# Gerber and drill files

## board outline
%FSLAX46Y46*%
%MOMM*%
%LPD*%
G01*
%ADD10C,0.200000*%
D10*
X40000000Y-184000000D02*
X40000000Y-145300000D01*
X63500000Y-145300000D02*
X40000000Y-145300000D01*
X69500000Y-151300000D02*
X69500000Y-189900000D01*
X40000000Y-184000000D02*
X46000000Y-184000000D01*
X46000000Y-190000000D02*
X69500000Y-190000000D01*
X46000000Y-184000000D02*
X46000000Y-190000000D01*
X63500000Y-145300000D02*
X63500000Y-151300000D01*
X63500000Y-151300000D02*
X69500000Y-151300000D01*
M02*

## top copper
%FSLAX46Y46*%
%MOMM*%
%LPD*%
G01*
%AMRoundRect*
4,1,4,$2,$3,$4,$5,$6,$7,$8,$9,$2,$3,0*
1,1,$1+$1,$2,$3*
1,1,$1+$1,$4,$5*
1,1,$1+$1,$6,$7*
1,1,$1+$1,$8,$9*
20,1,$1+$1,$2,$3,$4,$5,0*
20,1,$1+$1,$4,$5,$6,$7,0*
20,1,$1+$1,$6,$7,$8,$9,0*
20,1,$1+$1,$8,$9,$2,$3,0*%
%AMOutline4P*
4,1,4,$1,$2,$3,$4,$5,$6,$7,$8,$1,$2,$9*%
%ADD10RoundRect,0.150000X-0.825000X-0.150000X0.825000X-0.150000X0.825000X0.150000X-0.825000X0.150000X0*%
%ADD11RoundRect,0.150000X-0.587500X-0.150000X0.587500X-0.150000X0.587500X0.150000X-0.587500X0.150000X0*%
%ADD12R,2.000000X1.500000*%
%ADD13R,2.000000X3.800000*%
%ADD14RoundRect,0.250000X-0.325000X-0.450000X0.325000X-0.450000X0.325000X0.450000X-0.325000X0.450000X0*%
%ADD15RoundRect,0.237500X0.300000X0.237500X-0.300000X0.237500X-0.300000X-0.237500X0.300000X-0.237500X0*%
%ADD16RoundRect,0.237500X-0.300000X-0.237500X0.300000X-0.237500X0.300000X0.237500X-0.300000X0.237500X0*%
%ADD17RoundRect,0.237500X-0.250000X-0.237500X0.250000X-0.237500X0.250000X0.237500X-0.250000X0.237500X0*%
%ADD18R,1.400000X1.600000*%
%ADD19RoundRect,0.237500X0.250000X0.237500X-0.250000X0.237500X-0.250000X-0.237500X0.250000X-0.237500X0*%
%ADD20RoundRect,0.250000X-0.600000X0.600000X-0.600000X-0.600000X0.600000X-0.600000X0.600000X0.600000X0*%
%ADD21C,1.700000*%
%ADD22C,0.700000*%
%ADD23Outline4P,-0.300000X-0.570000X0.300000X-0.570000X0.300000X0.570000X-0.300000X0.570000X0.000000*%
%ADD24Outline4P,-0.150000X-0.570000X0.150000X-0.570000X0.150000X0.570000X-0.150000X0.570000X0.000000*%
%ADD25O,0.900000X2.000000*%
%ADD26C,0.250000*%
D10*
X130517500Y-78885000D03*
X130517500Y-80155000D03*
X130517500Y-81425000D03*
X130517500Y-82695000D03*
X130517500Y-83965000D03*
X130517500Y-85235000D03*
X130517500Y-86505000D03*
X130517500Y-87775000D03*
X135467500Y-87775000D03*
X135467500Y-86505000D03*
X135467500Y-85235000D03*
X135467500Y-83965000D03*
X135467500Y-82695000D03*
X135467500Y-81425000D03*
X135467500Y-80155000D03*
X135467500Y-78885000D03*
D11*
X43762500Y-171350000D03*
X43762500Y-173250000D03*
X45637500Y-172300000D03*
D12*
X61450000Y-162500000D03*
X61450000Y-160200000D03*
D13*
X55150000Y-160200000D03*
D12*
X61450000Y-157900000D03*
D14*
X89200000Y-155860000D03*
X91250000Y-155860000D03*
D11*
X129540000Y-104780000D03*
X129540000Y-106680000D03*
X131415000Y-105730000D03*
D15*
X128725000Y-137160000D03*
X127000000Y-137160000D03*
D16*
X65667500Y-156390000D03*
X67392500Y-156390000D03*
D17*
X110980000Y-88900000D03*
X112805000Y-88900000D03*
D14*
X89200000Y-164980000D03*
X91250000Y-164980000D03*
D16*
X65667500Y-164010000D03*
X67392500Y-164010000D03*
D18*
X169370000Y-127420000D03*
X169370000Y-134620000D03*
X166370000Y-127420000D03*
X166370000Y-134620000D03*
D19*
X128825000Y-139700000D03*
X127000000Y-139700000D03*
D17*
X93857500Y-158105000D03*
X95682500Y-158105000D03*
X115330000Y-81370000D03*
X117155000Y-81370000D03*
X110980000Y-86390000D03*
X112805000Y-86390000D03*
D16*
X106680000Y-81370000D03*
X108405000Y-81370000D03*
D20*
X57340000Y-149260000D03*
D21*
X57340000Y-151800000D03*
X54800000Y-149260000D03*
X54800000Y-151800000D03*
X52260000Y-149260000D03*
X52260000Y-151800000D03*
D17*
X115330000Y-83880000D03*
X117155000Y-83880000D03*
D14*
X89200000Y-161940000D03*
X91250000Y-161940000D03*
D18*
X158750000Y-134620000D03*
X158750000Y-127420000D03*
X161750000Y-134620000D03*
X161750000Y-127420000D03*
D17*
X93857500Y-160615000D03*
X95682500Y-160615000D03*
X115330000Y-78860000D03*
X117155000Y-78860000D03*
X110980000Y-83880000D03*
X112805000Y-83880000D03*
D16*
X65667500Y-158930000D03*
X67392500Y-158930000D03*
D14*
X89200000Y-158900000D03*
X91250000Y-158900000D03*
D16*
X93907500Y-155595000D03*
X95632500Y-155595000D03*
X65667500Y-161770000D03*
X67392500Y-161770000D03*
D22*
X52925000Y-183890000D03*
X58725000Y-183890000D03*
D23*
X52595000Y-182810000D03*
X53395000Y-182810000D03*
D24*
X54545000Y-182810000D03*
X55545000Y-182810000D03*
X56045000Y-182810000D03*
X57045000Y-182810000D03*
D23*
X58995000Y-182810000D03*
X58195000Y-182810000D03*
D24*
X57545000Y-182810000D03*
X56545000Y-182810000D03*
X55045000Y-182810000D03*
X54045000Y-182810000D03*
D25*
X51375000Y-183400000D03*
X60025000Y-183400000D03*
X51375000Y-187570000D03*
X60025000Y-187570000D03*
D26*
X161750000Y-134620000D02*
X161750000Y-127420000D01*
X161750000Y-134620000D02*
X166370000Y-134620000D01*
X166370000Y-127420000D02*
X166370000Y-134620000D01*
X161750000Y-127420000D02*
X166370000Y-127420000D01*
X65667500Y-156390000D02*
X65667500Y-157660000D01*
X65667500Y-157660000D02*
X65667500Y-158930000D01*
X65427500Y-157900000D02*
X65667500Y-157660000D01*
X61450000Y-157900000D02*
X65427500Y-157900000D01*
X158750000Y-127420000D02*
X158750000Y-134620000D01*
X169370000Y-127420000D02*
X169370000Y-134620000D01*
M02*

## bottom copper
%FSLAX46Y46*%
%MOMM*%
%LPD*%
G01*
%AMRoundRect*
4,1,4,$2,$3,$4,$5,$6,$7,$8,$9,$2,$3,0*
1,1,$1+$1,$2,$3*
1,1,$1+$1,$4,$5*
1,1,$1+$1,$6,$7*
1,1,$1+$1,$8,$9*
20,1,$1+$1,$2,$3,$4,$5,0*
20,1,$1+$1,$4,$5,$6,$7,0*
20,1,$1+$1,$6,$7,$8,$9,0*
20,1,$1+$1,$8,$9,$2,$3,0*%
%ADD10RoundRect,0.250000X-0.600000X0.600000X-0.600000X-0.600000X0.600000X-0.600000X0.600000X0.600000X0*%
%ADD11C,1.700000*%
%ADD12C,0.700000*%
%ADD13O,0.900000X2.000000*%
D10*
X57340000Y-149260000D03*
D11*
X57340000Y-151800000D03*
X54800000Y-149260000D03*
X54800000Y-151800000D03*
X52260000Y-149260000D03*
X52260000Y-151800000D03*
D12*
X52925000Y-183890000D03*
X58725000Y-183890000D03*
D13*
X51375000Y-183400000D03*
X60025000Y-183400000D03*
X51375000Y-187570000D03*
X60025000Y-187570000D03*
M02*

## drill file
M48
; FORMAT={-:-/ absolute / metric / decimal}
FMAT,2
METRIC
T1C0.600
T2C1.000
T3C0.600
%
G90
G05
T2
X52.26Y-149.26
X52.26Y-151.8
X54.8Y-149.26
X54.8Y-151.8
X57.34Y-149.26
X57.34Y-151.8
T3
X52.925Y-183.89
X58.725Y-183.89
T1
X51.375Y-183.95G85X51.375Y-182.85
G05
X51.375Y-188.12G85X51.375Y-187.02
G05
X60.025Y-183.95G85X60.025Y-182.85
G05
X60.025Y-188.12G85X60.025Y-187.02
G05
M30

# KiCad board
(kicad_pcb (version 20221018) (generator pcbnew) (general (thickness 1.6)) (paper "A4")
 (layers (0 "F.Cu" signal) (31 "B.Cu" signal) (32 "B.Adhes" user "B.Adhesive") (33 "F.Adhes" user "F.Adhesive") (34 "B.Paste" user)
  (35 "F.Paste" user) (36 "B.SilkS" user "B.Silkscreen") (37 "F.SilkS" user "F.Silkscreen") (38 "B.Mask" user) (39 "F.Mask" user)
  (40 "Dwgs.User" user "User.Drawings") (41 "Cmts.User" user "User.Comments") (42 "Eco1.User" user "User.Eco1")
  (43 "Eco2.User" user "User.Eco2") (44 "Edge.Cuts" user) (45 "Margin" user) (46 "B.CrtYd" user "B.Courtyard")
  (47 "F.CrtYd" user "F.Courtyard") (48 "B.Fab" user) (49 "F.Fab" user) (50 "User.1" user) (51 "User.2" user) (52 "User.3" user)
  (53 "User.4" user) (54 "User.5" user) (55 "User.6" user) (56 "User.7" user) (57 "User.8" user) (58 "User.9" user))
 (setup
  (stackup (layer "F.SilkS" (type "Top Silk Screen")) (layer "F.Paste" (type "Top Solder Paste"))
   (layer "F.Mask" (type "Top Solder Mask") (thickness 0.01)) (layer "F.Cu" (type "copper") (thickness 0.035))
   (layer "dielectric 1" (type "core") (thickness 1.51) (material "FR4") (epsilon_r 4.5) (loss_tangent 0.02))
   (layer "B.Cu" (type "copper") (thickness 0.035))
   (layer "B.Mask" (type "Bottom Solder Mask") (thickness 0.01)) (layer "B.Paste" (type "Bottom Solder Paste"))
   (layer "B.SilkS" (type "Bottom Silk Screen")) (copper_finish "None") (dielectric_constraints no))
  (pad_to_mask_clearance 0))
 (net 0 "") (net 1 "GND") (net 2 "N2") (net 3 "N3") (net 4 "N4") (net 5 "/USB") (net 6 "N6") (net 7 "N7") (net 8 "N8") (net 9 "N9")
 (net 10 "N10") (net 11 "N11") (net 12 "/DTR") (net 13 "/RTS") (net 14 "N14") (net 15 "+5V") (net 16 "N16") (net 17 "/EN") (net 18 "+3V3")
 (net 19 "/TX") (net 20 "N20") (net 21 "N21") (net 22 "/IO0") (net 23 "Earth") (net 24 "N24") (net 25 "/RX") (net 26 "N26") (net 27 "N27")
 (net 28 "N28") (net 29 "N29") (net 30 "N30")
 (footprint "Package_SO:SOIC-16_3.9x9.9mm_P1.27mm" (layer "F.Cu") (at 132.9925 83.33)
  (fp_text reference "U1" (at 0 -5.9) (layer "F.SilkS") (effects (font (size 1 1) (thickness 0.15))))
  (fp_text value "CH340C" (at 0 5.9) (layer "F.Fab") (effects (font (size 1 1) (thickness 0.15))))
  (pad "1" smd roundrect (at -2.475 -4.445) (size 1.95 0.6) (layers "F.Cu" "F.Paste" "F.Mask") (roundrect_rratio 0.25) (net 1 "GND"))
  (pad "2" smd roundrect (at -2.475 -3.175) (size 1.95 0.6) (layers "F.Cu" "F.Paste" "F.Mask") (roundrect_rratio 0.25) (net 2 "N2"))
  (pad "3" smd roundrect (at -2.475 -1.905) (size 1.95 0.6) (layers "F.Cu" "F.Paste" "F.Mask") (roundrect_rratio 0.25) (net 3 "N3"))
  (pad "4" smd roundrect (at -2.475 -0.635) (size 1.95 0.6) (layers "F.Cu" "F.Paste" "F.Mask") (roundrect_rratio 0.25) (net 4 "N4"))
  (pad "5" smd roundrect (at -2.475 0.635) (size 1.95 0.6) (layers "F.Cu" "F.Paste" "F.Mask") (roundrect_rratio 0.25) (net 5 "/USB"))
  (pad "6" smd roundrect (at -2.475 1.905) (size 1.95 0.6) (layers "F.Cu" "F.Paste" "F.Mask") (roundrect_rratio 0.25) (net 5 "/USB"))
  (pad "7" smd roundrect (at -2.475 3.175) (size 1.95 0.6) (layers "F.Cu" "F.Paste" "F.Mask") (roundrect_rratio 0.25) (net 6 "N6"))
  (pad "8" smd roundrect (at -2.475 4.445) (size 1.95 0.6) (layers "F.Cu" "F.Paste" "F.Mask") (roundrect_rratio 0.25) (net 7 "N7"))
  (pad "9" smd roundrect (at 2.475 4.445) (size 1.95 0.6) (layers "F.Cu" "F.Paste" "F.Mask") (roundrect_rratio 0.25) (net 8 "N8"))
  (pad "10" smd roundrect (at 2.475 3.175) (size 1.95 0.6) (layers "F.Cu" "F.Paste" "F.Mask") (roundrect_rratio 0.25) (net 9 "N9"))
  (pad "11" smd roundrect (at 2.475 1.905) (size 1.95 0.6) (layers "F.Cu" "F.Paste" "F.Mask") (roundrect_rratio 0.25) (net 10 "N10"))
  (pad "12" smd roundrect (at 2.475 0.635) (size 1.95 0.6) (layers "F.Cu" "F.Paste" "F.Mask") (roundrect_rratio 0.25) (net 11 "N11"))
  (pad "13" smd roundrect (at 2.475 -0.635) (size 1.95 0.6) (layers "F.Cu" "F.Paste" "F.Mask") (roundrect_rratio 0.25) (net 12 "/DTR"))
  (pad "14" smd roundrect (at 2.475 -1.905) (size 1.95 0.6) (layers "F.Cu" "F.Paste" "F.Mask") (roundrect_rratio 0.25) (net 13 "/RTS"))
  (pad "15" smd roundrect (at 2.475 -3.175) (size 1.95 0.6) (layers "F.Cu" "F.Paste" "F.Mask") (roundrect_rratio 0.25) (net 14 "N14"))
  (pad "16" smd roundrect (at 2.475 -4.445) (size 1.95 0.6) (layers "F.Cu" "F.Paste" "F.Mask") (roundrect_rratio 0.25) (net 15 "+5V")))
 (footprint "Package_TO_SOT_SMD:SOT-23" (layer "F.Cu") (at 44.7 172.3)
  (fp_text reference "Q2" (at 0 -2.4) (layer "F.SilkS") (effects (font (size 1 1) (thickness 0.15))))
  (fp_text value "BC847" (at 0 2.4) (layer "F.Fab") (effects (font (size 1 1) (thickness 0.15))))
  (pad "1" smd roundrect (at -0.9375 -0.95) (size 1.475 0.6) (layers "F.Cu" "F.Paste" "F.Mask") (roundrect_rratio 0.25) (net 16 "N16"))
  (pad "2" smd roundrect (at -0.9375 0.95) (size 1.475 0.6) (layers "F.Cu" "F.Paste" "F.Mask") (roundrect_rratio 0.25) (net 13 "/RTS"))
  (pad "3" smd roundrect (at 0.9375 0) (size 1.475 0.6) (layers "F.Cu" "F.Paste" "F.Mask") (roundrect_rratio 0.25) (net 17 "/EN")))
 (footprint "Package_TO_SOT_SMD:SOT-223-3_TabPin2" (layer "F.Cu") (at 58.3 160.2 180)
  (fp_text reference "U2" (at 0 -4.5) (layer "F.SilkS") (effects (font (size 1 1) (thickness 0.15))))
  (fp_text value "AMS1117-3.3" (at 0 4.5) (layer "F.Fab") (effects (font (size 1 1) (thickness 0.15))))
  (pad "1" smd rect (at -3.15 -2.3 180) (size 2 1.5) (layers "F.Cu" "F.Paste" "F.Mask") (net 1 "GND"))
  (pad "2" smd rect (at -3.15 0 180) (size 2 1.5) (layers "F.Cu" "F.Paste" "F.Mask") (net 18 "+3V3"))
  (pad "2" smd rect (at 3.15 0 180) (size 2 3.8) (layers "F.Cu" "F.Paste" "F.Mask") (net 18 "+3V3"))
  (pad "3" smd rect (at -3.15 2.3 180) (size 2 1.5) (layers "F.Cu" "F.Paste" "F.Mask") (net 15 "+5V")))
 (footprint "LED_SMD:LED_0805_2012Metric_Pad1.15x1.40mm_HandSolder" (layer "F.Cu") (at 90.225 155.86)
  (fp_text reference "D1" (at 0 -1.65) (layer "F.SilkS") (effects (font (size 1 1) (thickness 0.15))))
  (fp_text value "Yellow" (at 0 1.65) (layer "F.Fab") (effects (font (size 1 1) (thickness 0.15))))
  (pad "1" smd roundrect (at -1.025 0) (size 1.15 1.4) (layers "F.Cu" "F.Paste" "F.Mask") (roundrect_rratio 0.217391) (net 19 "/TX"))
  (pad "2" smd roundrect (at 1.025 0) (size 1.15 1.4) (layers "F.Cu" "F.Paste" "F.Mask") (roundrect_rratio 0.217391) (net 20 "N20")))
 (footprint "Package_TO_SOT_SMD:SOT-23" (layer "F.Cu") (at 130.4775 105.73)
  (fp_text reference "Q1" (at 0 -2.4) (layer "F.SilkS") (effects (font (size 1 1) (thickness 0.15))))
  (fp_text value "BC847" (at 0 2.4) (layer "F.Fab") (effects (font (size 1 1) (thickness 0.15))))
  (pad "1" smd roundrect (at -0.9375 -0.95) (size 1.475 0.6) (layers "F.Cu" "F.Paste" "F.Mask") (roundrect_rratio 0.25) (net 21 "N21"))
  (pad "2" smd roundrect (at -0.9375 0.95) (size 1.475 0.6) (layers "F.Cu" "F.Paste" "F.Mask") (roundrect_rratio 0.25) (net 12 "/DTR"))
  (pad "3" smd roundrect (at 0.9375 0) (size 1.475 0.6) (layers "F.Cu" "F.Paste" "F.Mask") (roundrect_rratio 0.25) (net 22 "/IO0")))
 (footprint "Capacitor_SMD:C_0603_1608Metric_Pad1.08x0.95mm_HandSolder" (layer "F.Cu") (at 127.8625 137.16 180)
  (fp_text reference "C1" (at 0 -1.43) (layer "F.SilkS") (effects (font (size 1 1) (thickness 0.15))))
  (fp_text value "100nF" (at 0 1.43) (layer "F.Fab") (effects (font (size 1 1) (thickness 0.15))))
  (pad "1" smd roundrect (at -0.8625 0 180) (size 1.075 0.95) (layers "F.Cu" "F.Paste" "F.Mask") (roundrect_rratio 0.25) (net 1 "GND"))
  (pad "2" smd roundrect (at 0.8625 0 180) (size 1.075 0.95) (layers "F.Cu" "F.Paste" "F.Mask") (roundrect_rratio 0.25) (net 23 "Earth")))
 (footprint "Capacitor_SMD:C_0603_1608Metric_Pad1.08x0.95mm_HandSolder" (layer "F.Cu") (at 66.53 156.39)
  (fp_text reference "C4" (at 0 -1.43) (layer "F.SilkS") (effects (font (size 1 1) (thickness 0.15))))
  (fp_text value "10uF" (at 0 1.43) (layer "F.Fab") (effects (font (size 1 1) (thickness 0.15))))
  (pad "1" smd roundrect (at -0.8625 0) (size 1.075 0.95) (layers "F.Cu" "F.Paste" "F.Mask") (roundrect_rratio 0.25) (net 15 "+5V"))
  (pad "2" smd roundrect (at 0.8625 0) (size 1.075 0.95) (layers "F.Cu" "F.Paste" "F.Mask") (roundrect_rratio 0.25) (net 1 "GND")))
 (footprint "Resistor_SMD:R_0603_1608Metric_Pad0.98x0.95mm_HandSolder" (layer "F.Cu") (at 111.8925 88.9)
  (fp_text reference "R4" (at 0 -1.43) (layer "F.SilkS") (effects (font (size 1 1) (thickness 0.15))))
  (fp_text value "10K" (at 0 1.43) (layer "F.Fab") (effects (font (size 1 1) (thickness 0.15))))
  (pad "1" smd roundrect (at -0.9125 0) (size 0.975 0.95) (layers "F.Cu" "F.Paste" "F.Mask") (roundrect_rratio 0.25) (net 22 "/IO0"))
  (pad "2" smd roundrect (at 0.9125 0) (size 0.975 0.95) (layers "F.Cu" "F.Paste" "F.Mask") (roundrect_rratio 0.25) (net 18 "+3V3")))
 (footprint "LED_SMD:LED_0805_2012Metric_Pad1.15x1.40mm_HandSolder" (layer "F.Cu") (at 90.225 164.98)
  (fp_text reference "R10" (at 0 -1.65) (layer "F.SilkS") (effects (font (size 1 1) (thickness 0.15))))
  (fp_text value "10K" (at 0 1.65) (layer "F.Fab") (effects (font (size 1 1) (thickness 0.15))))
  (pad "1" smd roundrect (at -1.025 0) (size 1.15 1.4) (layers "F.Cu" "F.Paste" "F.Mask") (roundrect_rratio 0.217391) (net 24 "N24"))
  (pad "2" smd roundrect (at 1.025 0) (size 1.15 1.4) (layers "F.Cu" "F.Paste" "F.Mask") (roundrect_rratio 0.217391) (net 18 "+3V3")))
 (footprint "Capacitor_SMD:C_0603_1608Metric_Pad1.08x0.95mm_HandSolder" (layer "F.Cu") (at 66.53 164.01)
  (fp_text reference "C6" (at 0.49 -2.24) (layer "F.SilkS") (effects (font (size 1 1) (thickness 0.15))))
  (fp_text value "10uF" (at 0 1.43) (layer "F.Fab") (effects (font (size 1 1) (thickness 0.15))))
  (pad "1" smd roundrect (at -0.8625 0) (size 1.075 0.95) (layers "F.Cu" "F.Paste" "F.Mask") (roundrect_rratio 0.25) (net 18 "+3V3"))
  (pad "2" smd roundrect (at 0.8625 0) (size 1.075 0.95) (layers "F.Cu" "F.Paste" "F.Mask") (roundrect_rratio 0.25) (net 1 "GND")))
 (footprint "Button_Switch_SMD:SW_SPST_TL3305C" (layer "F.Cu") (at 167.87 131.02 -90)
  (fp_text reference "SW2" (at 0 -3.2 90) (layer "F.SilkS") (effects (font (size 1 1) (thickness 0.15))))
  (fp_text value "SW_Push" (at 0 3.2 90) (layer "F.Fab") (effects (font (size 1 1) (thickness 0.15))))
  (pad "1" smd rect (at -3.6 -1.5 270) (size 1.6 1.4) (layers "F.Cu" "F.Paste" "F.Mask") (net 17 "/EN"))
  (pad "1" smd rect (at 3.6 -1.5 270) (size 1.6 1.4) (layers "F.Cu" "F.Paste" "F.Mask") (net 17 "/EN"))
  (pad "2" smd rect (at -3.6 1.5 270) (size 1.6 1.4) (layers "F.Cu" "F.Paste" "F.Mask") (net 1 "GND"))
  (pad "2" smd rect (at 3.6 1.5 270) (size 1.6 1.4) (layers "F.Cu" "F.Paste" "F.Mask") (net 1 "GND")))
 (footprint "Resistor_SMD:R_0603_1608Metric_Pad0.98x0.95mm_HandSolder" (layer "F.Cu") (at 127.9125 139.7 180)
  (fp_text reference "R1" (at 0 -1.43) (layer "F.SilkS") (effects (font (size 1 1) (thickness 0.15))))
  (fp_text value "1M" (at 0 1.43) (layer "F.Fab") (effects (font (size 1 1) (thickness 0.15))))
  (pad "1" smd roundrect (at -0.9125 0 180) (size 0.975 0.95) (layers "F.Cu" "F.Paste" "F.Mask") (roundrect_rratio 0.25) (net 1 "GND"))
  (pad "2" smd roundrect (at 0.9125 0 180) (size 0.975 0.95) (layers "F.Cu" "F.Paste" "F.Mask") (roundrect_rratio 0.25) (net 23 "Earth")))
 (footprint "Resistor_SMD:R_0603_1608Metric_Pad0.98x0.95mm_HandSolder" (layer "F.Cu") (at 94.77 158.105)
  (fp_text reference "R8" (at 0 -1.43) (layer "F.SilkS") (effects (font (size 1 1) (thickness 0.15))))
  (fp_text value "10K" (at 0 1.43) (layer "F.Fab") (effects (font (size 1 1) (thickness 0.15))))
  (pad "1" smd roundrect (at -0.9125 0) (size 0.975 0.95) (layers "F.Cu" "F.Paste" "F.Mask") (roundrect_rratio 0.25) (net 20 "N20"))
  (pad "2" smd roundrect (at 0.9125 0) (size 0.975 0.95) (layers "F.Cu" "F.Paste" "F.Mask") (roundrect_rratio 0.25) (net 18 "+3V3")))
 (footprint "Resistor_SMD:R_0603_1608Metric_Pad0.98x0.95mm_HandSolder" (layer "F.Cu") (at 116.2425 81.37)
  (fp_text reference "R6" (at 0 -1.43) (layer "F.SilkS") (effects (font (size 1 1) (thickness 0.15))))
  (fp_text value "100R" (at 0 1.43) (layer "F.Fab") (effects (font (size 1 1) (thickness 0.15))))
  (pad "1" smd roundrect (at -0.9125 0) (size 0.975 0.95) (layers "F.Cu" "F.Paste" "F.Mask") (roundrect_rratio 0.25) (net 2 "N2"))
  (pad "2" smd roundrect (at 0.9125 0) (size 0.975 0.95) (layers "F.Cu" "F.Paste" "F.Mask") (roundrect_rratio 0.25) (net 19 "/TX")))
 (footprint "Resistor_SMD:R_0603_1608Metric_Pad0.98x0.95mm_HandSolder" (layer "F.Cu") (at 111.8925 86.39)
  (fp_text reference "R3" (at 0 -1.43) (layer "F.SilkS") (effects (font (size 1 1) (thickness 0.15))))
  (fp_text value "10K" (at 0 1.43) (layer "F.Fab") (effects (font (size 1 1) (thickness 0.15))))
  (pad "1" smd roundrect (at -0.9125 0) (size 0.975 0.95) (layers "F.Cu" "F.Paste" "F.Mask") (roundrect_rratio 0.25) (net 12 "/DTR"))
  (pad "2" smd roundrect (at 0.9125 0) (size 0.975 0.95) (layers "F.Cu" "F.Paste" "F.Mask") (roundrect_rratio 0.25) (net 16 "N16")))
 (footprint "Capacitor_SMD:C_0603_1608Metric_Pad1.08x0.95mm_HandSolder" (layer "F.Cu") (at 107.5425 81.37)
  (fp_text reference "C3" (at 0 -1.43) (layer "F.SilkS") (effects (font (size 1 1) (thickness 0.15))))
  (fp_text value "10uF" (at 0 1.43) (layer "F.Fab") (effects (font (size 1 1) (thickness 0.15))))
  (pad "1" smd roundrect (at -0.8625 0) (size 1.075 0.95) (layers "F.Cu" "F.Paste" "F.Mask") (roundrect_rratio 0.25) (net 15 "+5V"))
  (pad "2" smd roundrect (at 0.8625 0) (size 1.075 0.95) (layers "F.Cu" "F.Paste" "F.Mask") (roundrect_rratio 0.25) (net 1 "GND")))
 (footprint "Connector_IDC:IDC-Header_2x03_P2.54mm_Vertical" (layer "F.Cu") (at 57.34 149.26 -90)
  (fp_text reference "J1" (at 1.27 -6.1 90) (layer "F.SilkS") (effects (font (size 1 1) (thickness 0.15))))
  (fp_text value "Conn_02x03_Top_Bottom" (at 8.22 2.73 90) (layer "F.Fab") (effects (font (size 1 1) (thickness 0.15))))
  (pad "1" thru_hole roundrect (at 0 0 270) (size 1.7 1.7) (drill 1) (layers "*.Cu" "*.Mask") (roundrect_rratio 0.147059) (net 18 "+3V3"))
  (pad "2" thru_hole circle (at 2.54 0 270) (size 1.7 1.7) (drill 1) (layers "*.Cu" "*.Mask") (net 22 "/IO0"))
  (pad "3" thru_hole circle (at 0 2.54 270) (size 1.7 1.7) (drill 1) (layers "*.Cu" "*.Mask") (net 1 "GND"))
  (pad "4" thru_hole circle (at 2.54 2.54 270) (size 1.7 1.7) (drill 1) (layers "*.Cu" "*.Mask") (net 19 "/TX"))
  (pad "5" thru_hole circle (at 0 5.08 270) (size 1.7 1.7) (drill 1) (layers "*.Cu" "*.Mask") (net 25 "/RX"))
  (pad "6" thru_hole circle (at 2.54 5.08 270) (size 1.7 1.7) (drill 1) (layers "*.Cu" "*.Mask") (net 17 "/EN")))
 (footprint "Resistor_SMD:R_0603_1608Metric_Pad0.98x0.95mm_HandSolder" (layer "F.Cu") (at 116.2425 83.88)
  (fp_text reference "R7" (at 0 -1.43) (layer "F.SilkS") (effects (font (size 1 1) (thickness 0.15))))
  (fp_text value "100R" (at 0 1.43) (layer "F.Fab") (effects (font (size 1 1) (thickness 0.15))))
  (pad "1" smd roundrect (at -0.9125 0) (size 0.975 0.95) (layers "F.Cu" "F.Paste" "F.Mask") (roundrect_rratio 0.25) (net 3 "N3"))
  (pad "2" smd roundrect (at 0.9125 0) (size 0.975 0.95) (layers "F.Cu" "F.Paste" "F.Mask") (roundrect_rratio 0.25) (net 25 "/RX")))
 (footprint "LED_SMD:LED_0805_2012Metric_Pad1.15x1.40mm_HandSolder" (layer "F.Cu") (at 90.225 161.94)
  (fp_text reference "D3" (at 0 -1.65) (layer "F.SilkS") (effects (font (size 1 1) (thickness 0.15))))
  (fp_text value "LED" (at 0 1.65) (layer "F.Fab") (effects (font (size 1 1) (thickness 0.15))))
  (pad "1" smd roundrect (at -1.025 0) (size 1.15 1.4) (layers "F.Cu" "F.Paste" "F.Mask") (roundrect_rratio 0.217391) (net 1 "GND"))
  (pad "2" smd roundrect (at 1.025 0) (size 1.15 1.4) (layers "F.Cu" "F.Paste" "F.Mask") (roundrect_rratio 0.217391) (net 24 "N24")))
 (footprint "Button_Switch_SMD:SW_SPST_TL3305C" (layer "F.Cu") (at 160.25 131.02 90)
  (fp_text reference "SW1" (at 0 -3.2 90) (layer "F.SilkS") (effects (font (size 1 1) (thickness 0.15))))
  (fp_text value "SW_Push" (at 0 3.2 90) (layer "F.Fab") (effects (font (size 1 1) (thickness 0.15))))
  (pad "1" smd rect (at -3.6 -1.5 90) (size 1.6 1.4) (layers "F.Cu" "F.Paste" "F.Mask") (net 22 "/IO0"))
  (pad "1" smd rect (at 3.6 -1.5 90) (size 1.6 1.4) (layers "F.Cu" "F.Paste" "F.Mask") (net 22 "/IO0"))
  (pad "2" smd rect (at -3.6 1.5 90) (size 1.6 1.4) (layers "F.Cu" "F.Paste" "F.Mask") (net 1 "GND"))
  (pad "2" smd rect (at 3.6 1.5 90) (size 1.6 1.4) (layers "F.Cu" "F.Paste" "F.Mask") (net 1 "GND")))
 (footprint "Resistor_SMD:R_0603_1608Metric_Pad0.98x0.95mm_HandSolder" (layer "F.Cu") (at 94.77 160.615)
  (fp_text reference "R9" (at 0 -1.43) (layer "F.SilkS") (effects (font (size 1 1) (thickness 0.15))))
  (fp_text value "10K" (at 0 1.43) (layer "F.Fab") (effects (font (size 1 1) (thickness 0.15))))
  (pad "1" smd roundrect (at -0.9125 0) (size 0.975 0.95) (layers "F.Cu" "F.Paste" "F.Mask") (roundrect_rratio 0.25) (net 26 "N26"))
  (pad "2" smd roundrect (at 0.9125 0) (size 0.975 0.95) (layers "F.Cu" "F.Paste" "F.Mask") (roundrect_rratio 0.25) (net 18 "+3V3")))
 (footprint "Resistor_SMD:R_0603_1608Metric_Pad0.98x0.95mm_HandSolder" (layer "F.Cu") (at 116.2425 78.86)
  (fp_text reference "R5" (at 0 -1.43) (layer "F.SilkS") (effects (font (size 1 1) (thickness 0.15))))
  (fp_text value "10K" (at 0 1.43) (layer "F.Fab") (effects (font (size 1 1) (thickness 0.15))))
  (pad "1" smd roundrect (at -0.9125 0) (size 0.975 0.95) (layers "F.Cu" "F.Paste" "F.Mask") (roundrect_rratio 0.25) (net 17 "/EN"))
  (pad "2" smd roundrect (at 0.9125 0) (size 0.975 0.95) (layers "F.Cu" "F.Paste" "F.Mask") (roundrect_rratio 0.25) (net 18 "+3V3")))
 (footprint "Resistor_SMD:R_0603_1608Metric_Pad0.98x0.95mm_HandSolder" (layer "F.Cu") (at 111.8925 83.88)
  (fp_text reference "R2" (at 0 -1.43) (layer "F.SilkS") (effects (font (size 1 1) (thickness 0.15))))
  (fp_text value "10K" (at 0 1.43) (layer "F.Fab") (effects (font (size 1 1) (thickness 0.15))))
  (pad "1" smd roundrect (at -0.9125 0) (size 0.975 0.95) (layers "F.Cu" "F.Paste" "F.Mask") (roundrect_rratio 0.25) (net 13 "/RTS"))
  (pad "2" smd roundrect (at 0.9125 0) (size 0.975 0.95) (layers "F.Cu" "F.Paste" "F.Mask") (roundrect_rratio 0.25) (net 21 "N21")))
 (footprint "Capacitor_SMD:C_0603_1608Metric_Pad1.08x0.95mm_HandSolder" (layer "F.Cu") (at 66.53 158.93)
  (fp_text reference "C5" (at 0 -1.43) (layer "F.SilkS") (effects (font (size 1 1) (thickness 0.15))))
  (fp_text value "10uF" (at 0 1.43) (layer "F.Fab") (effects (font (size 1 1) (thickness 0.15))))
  (pad "1" smd roundrect (at -0.8625 0) (size 1.075 0.95) (layers "F.Cu" "F.Paste" "F.Mask") (roundrect_rratio 0.25) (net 15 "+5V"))
  (pad "2" smd roundrect (at 0.8625 0) (size 1.075 0.95) (layers "F.Cu" "F.Paste" "F.Mask") (roundrect_rratio 0.25) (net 1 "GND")))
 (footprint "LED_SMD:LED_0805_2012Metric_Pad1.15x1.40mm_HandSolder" (layer "F.Cu") (at 90.225 158.9)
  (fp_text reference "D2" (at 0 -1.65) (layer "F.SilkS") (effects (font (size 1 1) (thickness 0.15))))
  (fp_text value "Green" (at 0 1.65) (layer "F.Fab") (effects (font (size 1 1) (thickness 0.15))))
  (pad "1" smd roundrect (at -1.025 0) (size 1.15 1.4) (layers "F.Cu" "F.Paste" "F.Mask") (roundrect_rratio 0.217391) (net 25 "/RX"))
  (pad "2" smd roundrect (at 1.025 0) (size 1.15 1.4) (layers "F.Cu" "F.Paste" "F.Mask") (roundrect_rratio 0.217391) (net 26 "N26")))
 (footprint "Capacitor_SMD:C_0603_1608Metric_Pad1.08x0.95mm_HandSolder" (layer "F.Cu") (at 94.77 155.595)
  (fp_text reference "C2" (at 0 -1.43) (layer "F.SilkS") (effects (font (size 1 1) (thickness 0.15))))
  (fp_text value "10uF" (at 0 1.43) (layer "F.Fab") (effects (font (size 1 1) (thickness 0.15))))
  (pad "1" smd roundrect (at -0.8625 0) (size 1.075 0.95) (layers "F.Cu" "F.Paste" "F.Mask") (roundrect_rratio 0.25) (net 4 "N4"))
  (pad "2" smd roundrect (at 0.8625 0) (size 1.075 0.95) (layers "F.Cu" "F.Paste" "F.Mask") (roundrect_rratio 0.25) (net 1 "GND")))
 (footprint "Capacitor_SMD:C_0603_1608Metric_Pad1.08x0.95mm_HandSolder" (layer "F.Cu") (at 66.53 161.77)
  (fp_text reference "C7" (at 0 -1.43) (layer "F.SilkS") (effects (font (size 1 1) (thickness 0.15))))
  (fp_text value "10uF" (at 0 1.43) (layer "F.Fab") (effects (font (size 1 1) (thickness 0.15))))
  (pad "1" smd roundrect (at -0.8625 0) (size 1.075 0.95) (layers "F.Cu" "F.Paste" "F.Mask") (roundrect_rratio 0.25) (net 18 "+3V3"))
  (pad "2" smd roundrect (at 0.8625 0) (size 1.075 0.95) (layers "F.Cu" "F.Paste" "F.Mask") (roundrect_rratio 0.25) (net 1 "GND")))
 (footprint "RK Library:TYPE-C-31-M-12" (layer "F.Cu") (at 55.325 178.7)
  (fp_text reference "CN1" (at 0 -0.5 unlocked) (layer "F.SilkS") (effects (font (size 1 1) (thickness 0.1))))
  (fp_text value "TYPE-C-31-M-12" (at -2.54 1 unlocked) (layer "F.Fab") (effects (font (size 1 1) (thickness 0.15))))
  (pad "" np_thru_hole circle (at -2.4 5.19) (size 0.7 0.7) (drill oval 0.6) (layers "*.Cu" "*.Mask"))
  (pad "" np_thru_hole circle (at 3.4 5.19) (size 0.7 0.7) (drill oval 0.6) (layers "*.Cu" "*.Mask"))
  (pad "A1/B12" smd trapezoid (at -2.73 4.11) (size 0.6 1.14) (layers "F.Cu" "F.Paste" "F.Mask") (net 1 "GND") (thermal_bridge_angle 45))
  (pad "A4/B9" smd trapezoid (at -1.93 4.11) (size 0.6 1.14) (layers "F.Cu" "F.Paste" "F.Mask") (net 15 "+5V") (thermal_bridge_angle 45))
  (pad "A5" smd trapezoid (at -0.78 4.11) (size 0.3 1.14) (layers "F.Cu" "F.Paste" "F.Mask") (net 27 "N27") (thermal_bridge_angle 45))
  (pad "A6" smd trapezoid (at 0.22 4.11) (size 0.3 1.14) (layers "F.Cu" "F.Paste" "F.Mask") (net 5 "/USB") (thermal_bridge_angle 45))
  (pad "A7" smd trapezoid (at 0.72 4.11) (size 0.3 1.14) (layers "F.Cu" "F.Paste" "F.Mask") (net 5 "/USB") (thermal_bridge_angle 45))
  (pad "A8" smd trapezoid (at 1.72 4.11) (size 0.3 1.14) (layers "F.Cu" "F.Paste" "F.Mask") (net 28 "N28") (thermal_bridge_angle 45))
  (pad "B1/A12" smd trapezoid (at 3.67 4.11) (size 0.6 1.14) (layers "F.Cu" "F.Paste" "F.Mask") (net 1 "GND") (thermal_bridge_angle 45))
  (pad "B4/A9" smd trapezoid (at 2.87 4.11) (size 0.6 1.14) (layers "F.Cu" "F.Paste" "F.Mask") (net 15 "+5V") (thermal_bridge_angle 45))
  (pad "B5" smd trapezoid (at 2.22 4.11) (size 0.3 1.14) (layers "F.Cu" "F.Paste" "F.Mask") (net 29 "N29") (thermal_bridge_angle 45))
  (pad "B6" smd trapezoid (at 1.22 4.11) (size 0.3 1.14) (layers "F.Cu" "F.Paste" "F.Mask") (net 5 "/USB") (thermal_bridge_angle 45))
  (pad "B7" smd trapezoid (at -0.28 4.11) (size 0.3 1.14) (layers "F.Cu" "F.Paste" "F.Mask") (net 5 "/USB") (thermal_bridge_angle 45))
  (pad "B8" smd trapezoid (at -1.28 4.11) (size 0.3 1.14) (layers "F.Cu" "F.Paste" "F.Mask") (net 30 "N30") (thermal_bridge_angle 45))
  (pad "S1" thru_hole oval (at -3.95 4.7 90) (size 2 0.9) (drill oval 1.7 0.6) (layers "*.Cu" "*.Mask") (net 23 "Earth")
   (thermal_bridge_angle 45))
  (pad "S2" thru_hole oval (at 4.7 4.7 90) (size 2 0.9) (drill oval 1.7 0.6) (layers "*.Cu" "*.Mask") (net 23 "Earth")
   (thermal_bridge_angle 45))
  (pad "S3" thru_hole oval (at -3.95 8.87 90) (size 2 0.9) (drill oval 1.7 0.6) (layers "*.Cu" "*.Mask") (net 23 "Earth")
   (thermal_bridge_angle 45))
  (pad "S4" thru_hole oval (at 4.7 8.87 90) (size 2 0.9) (drill oval 1.7 0.6) (layers "*.Cu" "*.Mask") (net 23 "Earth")
   (thermal_bridge_angle 45)))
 (gr_line (start 40 184) (end 40 145.3) (stroke (width 0.2) (type default)) (layer "Edge.Cuts"))
 (gr_line (start 63.5 145.3) (end 40 145.3) (stroke (width 0.2) (type default)) (layer "Edge.Cuts"))
 (gr_line (start 69.5 151.3) (end 69.5 189.9) (stroke (width 0.2) (type default)) (layer "Edge.Cuts"))
 (gr_line (start 40 184) (end 46 184) (stroke (width 0.2) (type default)) (layer "Edge.Cuts"))
 (gr_line (start 46 190) (end 69.5 190) (stroke (width 0.2) (type default)) (layer "Edge.Cuts"))
 (gr_line (start 46 184) (end 46 190) (stroke (width 0.2) (type default)) (layer "Edge.Cuts"))
 (gr_line (start 63.5 145.3) (end 63.5 151.3) (stroke (width 0.2) (type default)) (layer "Edge.Cuts"))
 (gr_line (start 63.5 151.3) (end 69.5 151.3) (stroke (width 0.2) (type default)) (layer "Edge.Cuts"))
 (segment (start 161.75 134.62) (end 161.75 127.42) (width 0.25) (layer "F.Cu") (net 1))
 (segment (start 161.75 134.62) (end 166.37 134.62) (width 0.25) (layer "F.Cu") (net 1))
 (segment (start 166.37 127.42) (end 166.37 134.62) (width 0.25) (layer "F.Cu") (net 1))
 (segment (start 161.75 127.42) (end 166.37 127.42) (width 0.25) (layer "F.Cu") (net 1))
 (segment (start 65.6675 156.39) (end 65.6675 157.66) (width 0.25) (layer "F.Cu") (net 15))
 (segment (start 65.6675 157.66) (end 65.6675 158.93) (width 0.25) (layer "F.Cu") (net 15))
 (segment (start 65.4275 157.9) (end 65.6675 157.66) (width 0.25) (layer "F.Cu") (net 15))
 (segment (start 61.45 157.9) (end 65.4275 157.9) (width 0.25) (layer "F.Cu") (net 15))
 (segment (start 158.75 127.42) (end 158.75 134.62) (width 0.25) (layer "F.Cu") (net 22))
 (segment (start 169.37 127.42) (end 169.37 134.62) (width 0.25) (layer "F.Cu") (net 17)))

